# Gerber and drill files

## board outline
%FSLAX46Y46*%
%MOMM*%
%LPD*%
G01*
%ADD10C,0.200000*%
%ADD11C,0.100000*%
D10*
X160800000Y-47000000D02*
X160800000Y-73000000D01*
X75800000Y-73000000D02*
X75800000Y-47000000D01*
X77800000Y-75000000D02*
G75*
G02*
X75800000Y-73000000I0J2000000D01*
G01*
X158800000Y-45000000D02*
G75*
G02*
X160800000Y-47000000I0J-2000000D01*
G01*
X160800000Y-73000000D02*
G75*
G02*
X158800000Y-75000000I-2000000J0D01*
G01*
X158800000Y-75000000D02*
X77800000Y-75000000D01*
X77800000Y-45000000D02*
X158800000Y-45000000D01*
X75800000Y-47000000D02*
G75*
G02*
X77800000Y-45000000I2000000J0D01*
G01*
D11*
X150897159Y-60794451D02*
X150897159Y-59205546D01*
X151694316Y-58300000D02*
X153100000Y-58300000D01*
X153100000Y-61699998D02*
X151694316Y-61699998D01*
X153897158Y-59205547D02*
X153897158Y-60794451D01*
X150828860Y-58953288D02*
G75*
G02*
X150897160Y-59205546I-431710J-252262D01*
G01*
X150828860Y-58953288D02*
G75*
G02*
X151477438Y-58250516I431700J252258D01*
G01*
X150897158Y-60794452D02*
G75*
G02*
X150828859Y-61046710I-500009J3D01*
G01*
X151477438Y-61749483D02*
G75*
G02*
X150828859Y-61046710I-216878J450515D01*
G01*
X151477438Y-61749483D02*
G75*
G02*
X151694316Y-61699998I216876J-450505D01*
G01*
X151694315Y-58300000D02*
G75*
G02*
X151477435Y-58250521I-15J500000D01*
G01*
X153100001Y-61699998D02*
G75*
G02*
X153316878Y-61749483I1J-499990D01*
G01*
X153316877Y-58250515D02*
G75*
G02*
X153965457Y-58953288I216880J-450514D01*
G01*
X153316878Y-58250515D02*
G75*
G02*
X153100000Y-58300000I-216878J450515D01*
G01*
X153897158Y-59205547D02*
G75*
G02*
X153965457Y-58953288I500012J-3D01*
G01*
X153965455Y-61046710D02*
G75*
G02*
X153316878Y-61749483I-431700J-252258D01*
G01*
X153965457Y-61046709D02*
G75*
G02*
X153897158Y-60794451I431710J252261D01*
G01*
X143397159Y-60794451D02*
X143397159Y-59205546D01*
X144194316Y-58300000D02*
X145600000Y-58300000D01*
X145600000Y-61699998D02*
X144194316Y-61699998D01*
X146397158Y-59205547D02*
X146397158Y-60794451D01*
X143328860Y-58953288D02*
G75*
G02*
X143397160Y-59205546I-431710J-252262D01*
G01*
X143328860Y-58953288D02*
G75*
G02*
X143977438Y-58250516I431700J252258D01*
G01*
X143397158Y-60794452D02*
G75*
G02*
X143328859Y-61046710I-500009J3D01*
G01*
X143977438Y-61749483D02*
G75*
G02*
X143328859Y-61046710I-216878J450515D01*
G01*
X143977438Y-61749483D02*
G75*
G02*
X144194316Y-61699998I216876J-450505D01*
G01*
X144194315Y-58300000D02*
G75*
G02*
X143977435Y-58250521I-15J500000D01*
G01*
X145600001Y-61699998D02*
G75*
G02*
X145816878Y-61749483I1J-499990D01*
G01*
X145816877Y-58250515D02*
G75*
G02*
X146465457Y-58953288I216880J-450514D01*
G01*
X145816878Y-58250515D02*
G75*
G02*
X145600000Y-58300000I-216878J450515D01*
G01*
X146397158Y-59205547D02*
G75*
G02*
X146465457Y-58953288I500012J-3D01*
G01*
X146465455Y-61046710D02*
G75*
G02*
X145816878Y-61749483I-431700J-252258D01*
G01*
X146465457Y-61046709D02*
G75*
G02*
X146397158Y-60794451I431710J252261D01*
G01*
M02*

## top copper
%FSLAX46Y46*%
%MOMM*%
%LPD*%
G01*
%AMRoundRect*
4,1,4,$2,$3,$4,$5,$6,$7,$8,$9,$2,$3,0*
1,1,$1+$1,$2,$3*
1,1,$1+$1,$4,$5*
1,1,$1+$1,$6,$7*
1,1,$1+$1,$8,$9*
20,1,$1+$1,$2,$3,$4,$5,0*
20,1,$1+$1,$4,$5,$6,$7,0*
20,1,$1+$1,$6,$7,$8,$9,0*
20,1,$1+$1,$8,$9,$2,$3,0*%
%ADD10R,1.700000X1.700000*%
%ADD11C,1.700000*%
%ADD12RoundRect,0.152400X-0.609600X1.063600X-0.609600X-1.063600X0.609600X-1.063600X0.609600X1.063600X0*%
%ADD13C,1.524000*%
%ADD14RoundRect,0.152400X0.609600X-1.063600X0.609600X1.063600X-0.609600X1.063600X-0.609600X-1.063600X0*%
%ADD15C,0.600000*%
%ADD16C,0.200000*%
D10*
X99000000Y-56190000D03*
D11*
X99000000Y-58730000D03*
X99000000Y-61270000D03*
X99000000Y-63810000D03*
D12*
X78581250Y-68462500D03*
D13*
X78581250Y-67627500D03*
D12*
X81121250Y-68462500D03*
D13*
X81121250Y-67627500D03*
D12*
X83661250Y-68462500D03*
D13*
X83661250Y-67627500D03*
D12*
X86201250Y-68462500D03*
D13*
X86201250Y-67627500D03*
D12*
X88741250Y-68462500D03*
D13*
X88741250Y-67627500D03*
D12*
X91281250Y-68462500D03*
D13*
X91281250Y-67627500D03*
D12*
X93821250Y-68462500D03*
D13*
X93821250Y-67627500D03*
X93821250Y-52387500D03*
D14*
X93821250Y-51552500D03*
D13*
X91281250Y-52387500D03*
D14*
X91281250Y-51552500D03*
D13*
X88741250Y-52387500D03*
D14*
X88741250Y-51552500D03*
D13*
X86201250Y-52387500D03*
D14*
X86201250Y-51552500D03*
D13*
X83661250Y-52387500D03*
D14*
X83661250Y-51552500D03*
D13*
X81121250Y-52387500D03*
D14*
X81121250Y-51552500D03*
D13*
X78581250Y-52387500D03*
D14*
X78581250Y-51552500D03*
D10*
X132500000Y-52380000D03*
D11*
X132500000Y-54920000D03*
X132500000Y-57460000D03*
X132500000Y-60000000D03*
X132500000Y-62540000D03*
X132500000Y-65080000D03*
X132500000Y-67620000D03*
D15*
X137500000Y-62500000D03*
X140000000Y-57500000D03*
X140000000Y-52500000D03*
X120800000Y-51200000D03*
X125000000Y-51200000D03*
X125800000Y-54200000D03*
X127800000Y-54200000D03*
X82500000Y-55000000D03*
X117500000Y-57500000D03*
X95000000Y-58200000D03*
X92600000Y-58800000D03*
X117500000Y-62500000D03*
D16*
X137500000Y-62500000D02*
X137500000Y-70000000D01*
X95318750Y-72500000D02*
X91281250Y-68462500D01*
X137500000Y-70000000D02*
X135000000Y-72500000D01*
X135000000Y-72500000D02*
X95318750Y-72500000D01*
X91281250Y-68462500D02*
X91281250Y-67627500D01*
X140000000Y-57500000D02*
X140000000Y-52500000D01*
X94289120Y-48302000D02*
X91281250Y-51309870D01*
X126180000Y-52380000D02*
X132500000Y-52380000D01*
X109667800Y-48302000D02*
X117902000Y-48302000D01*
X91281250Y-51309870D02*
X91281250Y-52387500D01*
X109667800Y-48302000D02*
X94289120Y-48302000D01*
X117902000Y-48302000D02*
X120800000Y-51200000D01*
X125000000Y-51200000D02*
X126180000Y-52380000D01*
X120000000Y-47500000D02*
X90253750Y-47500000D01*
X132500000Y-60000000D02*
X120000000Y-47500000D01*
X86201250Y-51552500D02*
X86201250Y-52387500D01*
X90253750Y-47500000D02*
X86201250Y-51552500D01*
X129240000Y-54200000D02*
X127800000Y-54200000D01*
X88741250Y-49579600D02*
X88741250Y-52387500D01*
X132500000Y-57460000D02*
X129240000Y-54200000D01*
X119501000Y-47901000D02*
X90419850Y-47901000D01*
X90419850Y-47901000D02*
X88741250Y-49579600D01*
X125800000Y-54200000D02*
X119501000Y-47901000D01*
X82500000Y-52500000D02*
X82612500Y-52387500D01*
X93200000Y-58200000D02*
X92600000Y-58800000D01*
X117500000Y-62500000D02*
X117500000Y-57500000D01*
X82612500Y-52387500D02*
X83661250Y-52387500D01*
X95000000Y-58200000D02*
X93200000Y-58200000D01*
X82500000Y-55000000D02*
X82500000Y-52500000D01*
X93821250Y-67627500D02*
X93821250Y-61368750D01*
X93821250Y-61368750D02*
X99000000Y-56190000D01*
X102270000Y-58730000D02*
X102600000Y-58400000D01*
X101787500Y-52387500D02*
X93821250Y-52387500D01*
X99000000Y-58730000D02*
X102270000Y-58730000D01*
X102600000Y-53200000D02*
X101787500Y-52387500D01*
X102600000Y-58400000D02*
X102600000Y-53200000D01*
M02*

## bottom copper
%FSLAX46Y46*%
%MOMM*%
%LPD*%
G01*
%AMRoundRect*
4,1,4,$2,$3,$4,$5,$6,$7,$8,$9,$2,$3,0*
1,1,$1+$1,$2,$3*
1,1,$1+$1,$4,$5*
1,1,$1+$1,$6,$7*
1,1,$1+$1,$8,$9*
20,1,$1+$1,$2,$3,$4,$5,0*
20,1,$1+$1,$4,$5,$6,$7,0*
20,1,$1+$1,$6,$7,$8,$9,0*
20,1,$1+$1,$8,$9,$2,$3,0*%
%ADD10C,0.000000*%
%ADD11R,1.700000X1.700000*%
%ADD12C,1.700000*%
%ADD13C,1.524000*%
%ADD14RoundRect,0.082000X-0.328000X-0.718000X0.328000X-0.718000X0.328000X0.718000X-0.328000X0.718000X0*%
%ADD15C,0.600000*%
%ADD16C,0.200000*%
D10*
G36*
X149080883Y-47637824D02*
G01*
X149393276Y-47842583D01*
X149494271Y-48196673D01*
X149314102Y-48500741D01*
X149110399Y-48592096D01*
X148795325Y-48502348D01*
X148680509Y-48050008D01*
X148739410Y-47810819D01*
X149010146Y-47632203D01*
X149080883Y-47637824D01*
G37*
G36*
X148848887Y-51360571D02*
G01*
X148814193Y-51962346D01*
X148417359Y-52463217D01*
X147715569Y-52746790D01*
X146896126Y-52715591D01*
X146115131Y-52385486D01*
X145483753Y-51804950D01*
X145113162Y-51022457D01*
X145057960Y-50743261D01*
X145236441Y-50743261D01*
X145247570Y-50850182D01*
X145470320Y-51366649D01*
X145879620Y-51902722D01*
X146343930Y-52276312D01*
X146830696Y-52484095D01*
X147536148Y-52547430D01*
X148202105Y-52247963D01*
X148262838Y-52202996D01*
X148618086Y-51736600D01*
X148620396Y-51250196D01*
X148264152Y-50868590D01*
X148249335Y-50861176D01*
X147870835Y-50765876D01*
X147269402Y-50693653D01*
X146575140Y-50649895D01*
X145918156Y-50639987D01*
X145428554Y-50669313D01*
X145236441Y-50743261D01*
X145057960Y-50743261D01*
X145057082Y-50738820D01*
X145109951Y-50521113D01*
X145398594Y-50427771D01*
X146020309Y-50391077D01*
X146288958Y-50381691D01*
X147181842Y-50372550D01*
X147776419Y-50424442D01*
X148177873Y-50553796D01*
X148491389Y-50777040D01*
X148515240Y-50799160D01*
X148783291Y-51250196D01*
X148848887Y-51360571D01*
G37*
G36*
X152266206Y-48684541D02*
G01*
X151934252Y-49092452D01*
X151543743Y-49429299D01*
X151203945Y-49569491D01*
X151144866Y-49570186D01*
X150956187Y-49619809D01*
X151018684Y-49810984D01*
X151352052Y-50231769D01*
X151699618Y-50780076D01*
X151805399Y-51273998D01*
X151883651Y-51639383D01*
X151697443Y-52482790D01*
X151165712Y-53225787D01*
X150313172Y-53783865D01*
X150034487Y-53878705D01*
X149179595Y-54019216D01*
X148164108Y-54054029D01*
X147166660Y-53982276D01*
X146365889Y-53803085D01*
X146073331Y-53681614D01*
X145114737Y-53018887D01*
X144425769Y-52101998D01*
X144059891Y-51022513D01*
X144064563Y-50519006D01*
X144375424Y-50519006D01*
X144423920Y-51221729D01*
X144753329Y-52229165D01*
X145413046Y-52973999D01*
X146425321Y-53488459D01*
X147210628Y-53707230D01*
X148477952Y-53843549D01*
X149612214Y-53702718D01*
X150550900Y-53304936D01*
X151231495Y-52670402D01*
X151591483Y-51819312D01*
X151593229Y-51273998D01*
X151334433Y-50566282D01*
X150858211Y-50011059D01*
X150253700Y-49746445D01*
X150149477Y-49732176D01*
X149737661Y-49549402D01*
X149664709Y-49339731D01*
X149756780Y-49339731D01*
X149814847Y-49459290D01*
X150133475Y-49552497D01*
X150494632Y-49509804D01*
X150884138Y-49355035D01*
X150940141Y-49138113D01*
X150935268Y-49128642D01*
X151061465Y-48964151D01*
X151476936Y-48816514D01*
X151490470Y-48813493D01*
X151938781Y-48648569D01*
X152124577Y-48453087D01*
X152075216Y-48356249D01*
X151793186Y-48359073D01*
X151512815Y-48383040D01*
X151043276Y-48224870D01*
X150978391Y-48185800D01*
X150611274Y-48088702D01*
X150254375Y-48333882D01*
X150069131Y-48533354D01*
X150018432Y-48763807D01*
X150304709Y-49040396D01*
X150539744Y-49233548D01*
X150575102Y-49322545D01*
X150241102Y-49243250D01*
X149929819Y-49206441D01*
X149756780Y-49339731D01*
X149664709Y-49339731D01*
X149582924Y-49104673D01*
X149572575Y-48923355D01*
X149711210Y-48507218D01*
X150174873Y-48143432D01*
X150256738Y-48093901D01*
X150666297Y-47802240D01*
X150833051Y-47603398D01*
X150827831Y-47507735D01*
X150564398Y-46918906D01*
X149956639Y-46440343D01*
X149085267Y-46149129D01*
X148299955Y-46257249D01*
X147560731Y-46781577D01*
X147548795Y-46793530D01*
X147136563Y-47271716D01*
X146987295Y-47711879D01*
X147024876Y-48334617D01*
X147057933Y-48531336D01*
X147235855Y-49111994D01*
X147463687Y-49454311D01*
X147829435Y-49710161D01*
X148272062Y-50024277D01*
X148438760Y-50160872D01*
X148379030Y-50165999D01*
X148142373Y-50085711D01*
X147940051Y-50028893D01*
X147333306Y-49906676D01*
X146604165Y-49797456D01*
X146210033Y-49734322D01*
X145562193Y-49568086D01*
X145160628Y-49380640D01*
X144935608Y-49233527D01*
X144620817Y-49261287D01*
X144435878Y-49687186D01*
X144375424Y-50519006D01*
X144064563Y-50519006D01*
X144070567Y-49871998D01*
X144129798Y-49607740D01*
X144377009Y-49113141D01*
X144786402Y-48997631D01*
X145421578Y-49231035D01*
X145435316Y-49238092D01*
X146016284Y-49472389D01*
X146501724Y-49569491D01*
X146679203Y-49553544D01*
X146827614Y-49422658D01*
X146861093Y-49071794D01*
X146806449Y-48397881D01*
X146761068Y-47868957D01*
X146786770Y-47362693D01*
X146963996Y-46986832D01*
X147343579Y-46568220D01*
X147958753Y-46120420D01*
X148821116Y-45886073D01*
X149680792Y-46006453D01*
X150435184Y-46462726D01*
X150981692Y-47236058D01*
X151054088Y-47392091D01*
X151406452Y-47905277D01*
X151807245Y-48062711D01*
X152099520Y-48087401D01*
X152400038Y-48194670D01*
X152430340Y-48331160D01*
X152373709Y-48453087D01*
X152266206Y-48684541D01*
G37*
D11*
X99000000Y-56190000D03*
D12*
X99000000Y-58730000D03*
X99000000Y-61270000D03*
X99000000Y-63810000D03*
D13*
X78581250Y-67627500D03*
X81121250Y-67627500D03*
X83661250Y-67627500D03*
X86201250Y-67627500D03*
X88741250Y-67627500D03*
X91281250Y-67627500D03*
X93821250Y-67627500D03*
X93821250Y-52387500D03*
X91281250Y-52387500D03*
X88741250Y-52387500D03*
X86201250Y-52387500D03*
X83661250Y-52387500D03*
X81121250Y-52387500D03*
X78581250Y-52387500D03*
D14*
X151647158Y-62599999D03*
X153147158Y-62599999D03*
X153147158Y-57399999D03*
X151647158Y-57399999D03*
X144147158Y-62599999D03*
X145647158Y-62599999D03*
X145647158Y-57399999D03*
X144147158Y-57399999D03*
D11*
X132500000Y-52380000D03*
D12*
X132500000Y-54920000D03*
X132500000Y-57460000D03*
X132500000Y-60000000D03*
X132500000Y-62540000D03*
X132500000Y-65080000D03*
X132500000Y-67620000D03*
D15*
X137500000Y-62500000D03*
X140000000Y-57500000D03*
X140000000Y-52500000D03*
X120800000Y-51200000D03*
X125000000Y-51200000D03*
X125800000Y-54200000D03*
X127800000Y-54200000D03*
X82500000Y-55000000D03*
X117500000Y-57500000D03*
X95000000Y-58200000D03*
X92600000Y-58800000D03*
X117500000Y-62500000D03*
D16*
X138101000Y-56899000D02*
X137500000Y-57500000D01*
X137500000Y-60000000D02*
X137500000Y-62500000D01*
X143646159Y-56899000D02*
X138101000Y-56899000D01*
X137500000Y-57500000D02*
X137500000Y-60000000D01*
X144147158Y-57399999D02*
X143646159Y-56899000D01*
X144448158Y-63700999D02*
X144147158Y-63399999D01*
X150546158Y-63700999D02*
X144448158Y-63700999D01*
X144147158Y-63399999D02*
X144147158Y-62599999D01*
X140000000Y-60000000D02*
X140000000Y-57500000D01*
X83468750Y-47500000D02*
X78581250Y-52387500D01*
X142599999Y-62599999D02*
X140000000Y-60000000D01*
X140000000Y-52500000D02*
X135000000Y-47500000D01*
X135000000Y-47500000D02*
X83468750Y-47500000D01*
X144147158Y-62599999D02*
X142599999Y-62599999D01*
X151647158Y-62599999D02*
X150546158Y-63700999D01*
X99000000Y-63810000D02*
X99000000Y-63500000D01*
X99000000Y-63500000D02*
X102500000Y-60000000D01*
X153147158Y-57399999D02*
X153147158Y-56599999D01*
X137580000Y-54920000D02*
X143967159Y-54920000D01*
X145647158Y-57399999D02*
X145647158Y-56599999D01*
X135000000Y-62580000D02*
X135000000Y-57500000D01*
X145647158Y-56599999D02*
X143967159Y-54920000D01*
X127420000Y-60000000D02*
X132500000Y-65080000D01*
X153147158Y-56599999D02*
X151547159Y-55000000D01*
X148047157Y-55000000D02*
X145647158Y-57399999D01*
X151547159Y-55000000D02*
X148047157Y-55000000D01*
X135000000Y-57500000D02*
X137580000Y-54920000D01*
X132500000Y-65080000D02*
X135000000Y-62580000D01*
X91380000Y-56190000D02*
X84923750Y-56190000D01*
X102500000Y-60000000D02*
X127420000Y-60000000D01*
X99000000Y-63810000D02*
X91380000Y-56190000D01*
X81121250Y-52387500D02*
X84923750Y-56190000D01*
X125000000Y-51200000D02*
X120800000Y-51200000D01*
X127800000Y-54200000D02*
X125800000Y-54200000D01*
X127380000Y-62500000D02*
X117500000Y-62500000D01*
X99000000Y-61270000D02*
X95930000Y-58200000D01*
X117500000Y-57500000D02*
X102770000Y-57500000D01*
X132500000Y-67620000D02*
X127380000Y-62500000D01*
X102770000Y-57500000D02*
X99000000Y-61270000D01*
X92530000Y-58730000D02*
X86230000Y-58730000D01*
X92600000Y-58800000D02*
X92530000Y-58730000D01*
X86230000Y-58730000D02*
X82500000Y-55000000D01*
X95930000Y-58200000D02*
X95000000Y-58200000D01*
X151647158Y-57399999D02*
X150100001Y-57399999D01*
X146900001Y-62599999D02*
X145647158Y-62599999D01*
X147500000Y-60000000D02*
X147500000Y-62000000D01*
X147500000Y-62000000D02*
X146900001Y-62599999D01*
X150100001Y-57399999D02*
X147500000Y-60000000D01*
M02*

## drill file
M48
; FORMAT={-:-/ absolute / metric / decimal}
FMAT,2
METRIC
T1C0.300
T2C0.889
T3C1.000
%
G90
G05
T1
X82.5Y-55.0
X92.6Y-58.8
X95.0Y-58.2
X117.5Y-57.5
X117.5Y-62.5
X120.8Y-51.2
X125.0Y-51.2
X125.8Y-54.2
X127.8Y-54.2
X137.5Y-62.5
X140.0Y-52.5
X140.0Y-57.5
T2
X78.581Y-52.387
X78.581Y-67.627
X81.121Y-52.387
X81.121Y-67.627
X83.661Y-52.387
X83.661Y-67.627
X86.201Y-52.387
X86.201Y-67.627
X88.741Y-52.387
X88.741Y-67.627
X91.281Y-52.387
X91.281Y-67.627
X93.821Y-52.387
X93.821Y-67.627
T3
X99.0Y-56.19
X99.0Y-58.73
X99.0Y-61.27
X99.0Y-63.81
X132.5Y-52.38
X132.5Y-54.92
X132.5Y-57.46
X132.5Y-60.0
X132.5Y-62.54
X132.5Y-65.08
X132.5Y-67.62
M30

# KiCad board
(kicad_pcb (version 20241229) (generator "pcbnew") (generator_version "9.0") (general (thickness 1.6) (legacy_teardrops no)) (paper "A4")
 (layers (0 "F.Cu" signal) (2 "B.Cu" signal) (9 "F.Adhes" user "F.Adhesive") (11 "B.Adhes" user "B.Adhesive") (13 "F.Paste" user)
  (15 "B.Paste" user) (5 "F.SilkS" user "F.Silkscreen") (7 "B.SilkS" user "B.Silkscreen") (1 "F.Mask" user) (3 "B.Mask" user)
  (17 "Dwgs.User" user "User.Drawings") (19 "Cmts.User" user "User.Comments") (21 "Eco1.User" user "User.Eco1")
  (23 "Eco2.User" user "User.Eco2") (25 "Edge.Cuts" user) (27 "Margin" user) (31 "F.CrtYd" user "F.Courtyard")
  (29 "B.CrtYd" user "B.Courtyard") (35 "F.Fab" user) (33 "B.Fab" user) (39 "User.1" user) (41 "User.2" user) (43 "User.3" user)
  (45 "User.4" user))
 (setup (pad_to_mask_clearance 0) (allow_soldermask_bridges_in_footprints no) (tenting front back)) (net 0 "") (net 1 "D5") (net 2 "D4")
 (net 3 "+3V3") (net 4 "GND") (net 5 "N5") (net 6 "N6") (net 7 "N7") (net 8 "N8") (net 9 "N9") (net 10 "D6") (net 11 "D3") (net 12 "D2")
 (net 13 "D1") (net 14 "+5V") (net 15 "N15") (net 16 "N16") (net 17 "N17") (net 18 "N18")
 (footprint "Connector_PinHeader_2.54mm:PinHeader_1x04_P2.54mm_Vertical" (layer "F.Cu") (at 99 56.19)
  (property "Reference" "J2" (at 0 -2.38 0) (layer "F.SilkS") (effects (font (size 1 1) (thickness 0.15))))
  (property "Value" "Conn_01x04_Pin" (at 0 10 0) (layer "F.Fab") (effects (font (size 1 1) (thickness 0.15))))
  (pad "1" thru_hole rect (at 0 0) (size 1.7 1.7) (drill 1) (layers "*.Cu" "*.Mask") (remove_unused_layers no) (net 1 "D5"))
  (pad "2" thru_hole circle (at 0 2.54) (size 1.7 1.7) (drill 1) (layers "*.Cu" "*.Mask") (remove_unused_layers no) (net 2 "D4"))
  (pad "3" thru_hole circle (at 0 5.08) (size 1.7 1.7) (drill 1) (layers "*.Cu" "*.Mask") (remove_unused_layers no) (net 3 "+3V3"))
  (pad "4" thru_hole circle (at 0 7.62) (size 1.7 1.7) (drill 1) (layers "*.Cu" "*.Mask") (remove_unused_layers no) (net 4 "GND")))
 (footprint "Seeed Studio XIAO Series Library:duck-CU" (layer "F.Cu") (at 148.25 50)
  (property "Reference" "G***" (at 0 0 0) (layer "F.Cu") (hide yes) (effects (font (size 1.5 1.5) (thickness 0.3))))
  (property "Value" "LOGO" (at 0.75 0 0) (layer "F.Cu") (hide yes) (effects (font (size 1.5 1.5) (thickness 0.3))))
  (fp_poly
   (pts (xy 0.48941 -2.189181) (xy 0.430509 -1.949992) (xy 0.545325 -1.497652) (xy 0.860399 -1.407904) (xy 1.064102 -1.499259)
    (xy 1.244271 -1.803327) (xy 1.143276 -2.157417) (xy 0.830883 -2.362176) (xy 0.760146 -2.367797))
   (stroke (width 0) (type solid)) (fill yes) (layer "B.Cu"))
  (fp_poly
   (pts (xy -1.961042 0.381691) (xy -2.229691 0.391077) (xy -2.851406 0.427771) (xy -3.140049 0.521113) (xy -3.192918 0.73882)
    (xy -3.136838 1.022457) (xy -2.766247 1.80495) (xy -2.134869 2.385486) (xy -1.353874 2.715591) (xy -0.534431 2.74679)
    (xy 0.167359 2.463217) (xy 0.564193 1.962346) (xy 0.598887 1.360571) (xy 0.533291 1.250196) (xy 0.370396 1.250196) (xy 0.368086 1.7366)
    (xy 0.012838 2.202996) (xy -0.047895 2.247963) (xy -0.713852 2.54743) (xy -1.419304 2.484095) (xy -1.90607 2.276312)
    (xy -2.37038 1.902722) (xy -2.77968 1.366649) (xy -3.00243 0.850182) (xy -3.013559 0.743261) (xy -2.821446 0.669313)
    (xy -2.331844 0.639987) (xy -1.67486 0.649895) (xy -0.980598 0.693653) (xy -0.379165 0.765876) (xy -0.000665 0.861176)
    (xy 0.014152 0.86859) (xy 0.370396 1.250196) (xy 0.533291 1.250196) (xy 0.26524 0.79916) (xy 0.241389 0.77704) (xy -0.072127 0.553796)
    (xy -0.473581 0.424442) (xy -1.068158 0.37255))
   (stroke (width 0) (type solid)) (fill yes) (layer "B.Cu"))
  (fp_poly
   (pts (xy -0.291247 -3.87958) (xy -0.906421 -3.43178) (xy -1.286004 -3.013168) (xy -1.46323 -2.637307) (xy -1.488932 -2.131043)
    (xy -1.443551 -1.602119) (xy -1.388907 -0.928206) (xy -1.422386 -0.577342) (xy -1.570797 -0.446456) (xy -1.748276 -0.430509)
    (xy -2.233716 -0.527611) (xy -2.814684 -0.761908) (xy -2.828422 -0.768965) (xy -3.463598 -1.002369) (xy -3.872991 -0.886859)
    (xy -4.120202 -0.39226) (xy -4.179433 -0.128002) (xy -4.190109 1.022513) (xy -3.824231 2.101998) (xy -3.135263 3.018887)
    (xy -2.176669 3.681614) (xy -1.884111 3.803085) (xy -1.08334 3.982276) (xy -0.085892 4.054029) (xy 0.929595 4.019216)
    (xy 1.784487 3.878705) (xy 2.063172 3.783865) (xy 2.915712 3.225787) (xy 3.447443 2.48279) (xy 3.633651 1.639383) (xy 3.555399 1.273998)
    (xy 3.343229 1.273998) (xy 3.341483 1.819312) (xy 2.981495 2.670402) (xy 2.3009 3.304936) (xy 1.362214 3.702718) (xy 0.227952 3.843549)
    (xy -1.039372 3.70723) (xy -1.824679 3.488459) (xy -2.836954 2.973999) (xy -3.496671 2.229165) (xy -3.82608 1.221729)
    (xy -3.874576 0.519006) (xy -3.814122 -0.312814) (xy -3.629183 -0.738713) (xy -3.314392 -0.766473) (xy -3.089372 -0.61936)
    (xy -2.687807 -0.431914) (xy -2.039967 -0.265678) (xy -1.645835 -0.202544) (xy -0.916694 -0.093324) (xy -0.309949 0.028893)
    (xy -0.107627 0.085711) (xy 0.12903 0.165999) (xy 0.18876 0.160872) (xy 0.022062 0.024277) (xy -0.420565 -0.289839)
    (xy -0.786313 -0.545689) (xy -1.014145 -0.888006) (xy -1.192067 -1.468664) (xy -1.225124 -1.665383) (xy -1.262705 -2.288121)
    (xy -1.113437 -2.728284) (xy -0.701205 -3.20647) (xy -0.689269 -3.218423) (xy 0.049955 -3.742751) (xy 0.835267 -3.850871)
    (xy 1.706639 -3.559657) (xy 2.314398 -3.081094) (xy 2.577831 -2.492265) (xy 2.583051 -2.396602) (xy 2.416297 -2.19776)
    (xy 2.006738 -1.906099) (xy 1.924873 -1.856568) (xy 1.46121 -1.492782) (xy 1.322575 -1.076645) (xy 1.332924 -0.895327)
    (xy 1.487661 -0.450598) (xy 1.899477 -0.267824) (xy 2.0037 -0.253555) (xy 2.608211 0.011059) (xy 3.084433 0.566282)
    (xy 3.343229 1.273998) (xy 3.555399 1.273998) (xy 3.449618 0.780076) (xy 3.102052 0.231769) (xy 2.768684 -0.189016)
    (xy 2.706187 -0.380191) (xy 2.894866 -0.429814) (xy 2.953945 -0.430509) (xy 3.293743 -0.570701) (xy 3.684252 -0.907548)
    (xy 4.016206 -1.315459) (xy 4.123709 -1.546913) (xy 3.874577 -1.546913) (xy 3.688781 -1.351431) (xy 3.24047 -1.186507)
    (xy 3.226936 -1.183486) (xy 2.811465 -1.035849) (xy 2.685268 -0.871358) (xy 2.690141 -0.861887) (xy 2.634138 -0.644965)
    (xy 2.244632 -0.490196) (xy 1.883475 -0.447503) (xy 1.564847 -0.54071) (xy 1.50678 -0.660269) (xy 1.679819 -0.793559)
    (xy 1.991102 -0.75675) (xy 2.325102 -0.677455) (xy 2.289744 -0.766452) (xy 2.054709 -0.959604) (xy 1.768432 -1.236193)
    (xy 1.819131 -1.466646) (xy 2.004375 -1.666118) (xy 2.361274 -1.911298) (xy 2.728391 -1.8142) (xy 2.793276 -1.77513)
    (xy 3.262815 -1.61696) (xy 3.543186 -1.640927) (xy 3.825216 -1.643751) (xy 3.874577 -1.546913) (xy 4.123709 -1.546913)
    (xy 4.18034 -1.66884) (xy 4.150038 -1.80533) (xy 3.84952 -1.912599) (xy 3.557245 -1.937289) (xy 3.156452 -2.094723)
    (xy 2.804088 -2.607909) (xy 2.731692 -2.763942) (xy 2.185184 -3.537274) (xy 1.430792 -3.993547) (xy 0.571116 -4.113927))
   (stroke (width 0) (type solid)) (fill yes) (layer "B.Cu")))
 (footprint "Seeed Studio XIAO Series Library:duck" (layer "F.Cu") (at 148 50)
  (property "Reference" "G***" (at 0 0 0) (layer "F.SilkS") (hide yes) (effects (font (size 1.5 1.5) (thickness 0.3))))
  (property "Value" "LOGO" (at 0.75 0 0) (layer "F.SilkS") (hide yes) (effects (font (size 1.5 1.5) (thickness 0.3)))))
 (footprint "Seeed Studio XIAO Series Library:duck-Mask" (layer "F.Cu") (at 148.25 50)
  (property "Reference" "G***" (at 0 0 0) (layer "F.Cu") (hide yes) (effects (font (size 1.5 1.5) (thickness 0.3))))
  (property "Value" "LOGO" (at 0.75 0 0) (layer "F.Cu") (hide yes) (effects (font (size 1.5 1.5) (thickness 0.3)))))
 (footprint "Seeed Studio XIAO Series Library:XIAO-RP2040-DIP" (layer "F.Cu") (at 86.20125 60.0075 90)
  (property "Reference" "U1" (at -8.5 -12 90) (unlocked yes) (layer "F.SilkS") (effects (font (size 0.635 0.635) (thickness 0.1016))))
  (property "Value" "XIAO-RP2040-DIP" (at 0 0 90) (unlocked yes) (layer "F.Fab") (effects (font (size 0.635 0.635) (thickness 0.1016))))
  (pad "1" smd roundrect (at -8.455 -7.62 270) (size 2.432 1.524) (layers "F.Cu" "F.Mask") (roundrect_rratio 0.1) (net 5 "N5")
   (thermal_bridge_angle 45))
  (pad "1" thru_hole circle (at -7.62 -7.62 270) (size 1.524 1.524) (drill 0.889) (layers "*.Cu" "*.Mask") (remove_unused_layers no)
   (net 5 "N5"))
  (pad "2" smd roundrect (at -8.455 -5.08 270) (size 2.432 1.524) (layers "F.Cu" "F.Mask") (roundrect_rratio 0.1) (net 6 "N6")
   (thermal_bridge_angle 45))
  (pad "2" thru_hole circle (at -7.62 -5.08 270) (size 1.524 1.524) (drill 0.889) (layers "*.Cu" "*.Mask") (remove_unused_layers no)
   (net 6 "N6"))
  (pad "3" smd roundrect (at -8.455 -2.54 270) (size 2.432 1.524) (layers "F.Cu" "F.Mask") (roundrect_rratio 0.1) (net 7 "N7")
   (thermal_bridge_angle 45))
  (pad "3" thru_hole circle (at -7.62 -2.54 270) (size 1.524 1.524) (drill 0.889) (layers "*.Cu" "*.Mask") (remove_unused_layers no)
   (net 7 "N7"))
  (pad "4" smd roundrect (at -8.455 0 270) (size 2.432 1.524) (layers "F.Cu" "F.Mask") (roundrect_rratio 0.1) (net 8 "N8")
   (thermal_bridge_angle 45))
  (pad "4" thru_hole circle (at -7.62 0 270) (size 1.524 1.524) (drill 0.889) (layers "*.Cu" "*.Mask") (remove_unused_layers no)
   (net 8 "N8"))
  (pad "5" smd roundrect (at -8.455 2.54 270) (size 2.432 1.524) (layers "F.Cu" "F.Mask") (roundrect_rratio 0.1) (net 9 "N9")
   (thermal_bridge_angle 45))
  (pad "5" thru_hole circle (at -7.62 2.54 270) (size 1.524 1.524) (drill 0.889) (layers "*.Cu" "*.Mask") (remove_unused_layers no)
   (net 9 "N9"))
  (pad "6" smd roundrect (at -8.455 5.08 270) (size 2.432 1.524) (layers "F.Cu" "F.Mask") (roundrect_rratio 0.1) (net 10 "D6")
   (thermal_bridge_angle 45))
  (pad "6" thru_hole circle (at -7.62 5.08 270) (size 1.524 1.524) (drill 0.889) (layers "*.Cu" "*.Mask") (remove_unused_layers no)
   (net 10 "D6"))
  (pad "7" smd roundrect (at -8.455 7.62 270) (size 2.432 1.524) (layers "F.Cu" "F.Mask") (roundrect_rratio 0.1) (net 1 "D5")
   (thermal_bridge_angle 45))
  (pad "7" thru_hole circle (at -7.62 7.62 270) (size 1.524 1.524) (drill 0.889) (layers "*.Cu" "*.Mask") (remove_unused_layers no)
   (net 1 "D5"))
  (pad "8" thru_hole circle (at 7.62 7.62 90) (size 1.524 1.524) (drill 0.889) (layers "*.Cu" "*.Mask") (remove_unused_layers no)
   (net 2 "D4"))
  (pad "8" smd roundrect (at 8.455 7.62 90) (size 2.432 1.524) (layers "F.Cu" "F.Mask") (roundrect_rratio 0.1) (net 2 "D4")
   (thermal_bridge_angle 45))
  (pad "9" thru_hole circle (at 7.62 5.08 90) (size 1.524 1.524) (drill 0.889) (layers "*.Cu" "*.Mask") (remove_unused_layers no)
   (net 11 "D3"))
  (pad "9" smd roundrect (at 8.455 5.08 90) (size 2.432 1.524) (layers "F.Cu" "F.Mask") (roundrect_rratio 0.1) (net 11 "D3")
   (thermal_bridge_angle 45))
  (pad "10" thru_hole circle (at 7.62 2.54 90) (size 1.524 1.524) (drill 0.889) (layers "*.Cu" "*.Mask") (remove_unused_layers no)
   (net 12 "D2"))
  (pad "10" smd roundrect (at 8.455 2.54 90) (size 2.432 1.524) (layers "F.Cu" "F.Mask") (roundrect_rratio 0.1) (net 12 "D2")
   (thermal_bridge_angle 45))
  (pad "11" thru_hole circle (at 7.62 0 90) (size 1.524 1.524) (drill 0.889) (layers "*.Cu" "*.Mask") (remove_unused_layers no)
   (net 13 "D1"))
  (pad "11" smd roundrect (at 8.455 0 90) (size 2.432 1.524) (layers "F.Cu" "F.Mask") (roundrect_rratio 0.1) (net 13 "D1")
   (thermal_bridge_angle 45))
  (pad "12" thru_hole circle (at 7.62 -2.54 90) (size 1.524 1.524) (drill 0.889) (layers "*.Cu" "*.Mask") (remove_unused_layers no)
   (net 3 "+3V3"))
  (pad "12" smd roundrect (at 8.455 -2.54 90) (size 2.432 1.524) (layers "F.Cu" "F.Mask") (roundrect_rratio 0.1) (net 3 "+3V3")
   (thermal_bridge_angle 45))
  (pad "13" thru_hole circle (at 7.62 -5.08 90) (size 1.524 1.524) (drill 0.889) (layers "*.Cu" "*.Mask") (remove_unused_layers no)
   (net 4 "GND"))
  (pad "13" smd roundrect (at 8.455 -5.08 90) (size 2.432 1.524) (layers "F.Cu" "F.Mask") (roundrect_rratio 0.1) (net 4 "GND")
   (thermal_bridge_angle 45))
  (pad "14" thru_hole circle (at 7.62 -7.62 90) (size 1.524 1.524) (drill 0.889) (layers "*.Cu" "*.Mask") (remove_unused_layers no)
   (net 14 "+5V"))
  (pad "14" smd roundrect (at 8.455 -7.62 90) (size 2.432 1.524) (layers "F.Cu" "F.Mask") (roundrect_rratio 0.1) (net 14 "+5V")
   (thermal_bridge_angle 45)))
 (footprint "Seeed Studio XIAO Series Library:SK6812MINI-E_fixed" (layer "F.Cu") (at 152.5 60 90)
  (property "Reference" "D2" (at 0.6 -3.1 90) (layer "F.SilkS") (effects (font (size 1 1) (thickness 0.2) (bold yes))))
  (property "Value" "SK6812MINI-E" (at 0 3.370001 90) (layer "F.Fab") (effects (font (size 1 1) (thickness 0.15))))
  (fp_line (start -0.794451 -1.602841) (end 0.794454 -1.602841) (stroke (width 0.1) (type solid)) (layer "Edge.Cuts"))
  (fp_line (start 1.7 -0.805684) (end 1.7 0.6) (stroke (width 0.1) (type solid)) (layer "Edge.Cuts"))
  (fp_line (start -1.699998 0.6) (end -1.699998 -0.805684) (stroke (width 0.1) (type solid)) (layer "Edge.Cuts"))
  (fp_line (start 0.794453 1.397158) (end -0.794451 1.397158) (stroke (width 0.1) (type solid)) (layer "Edge.Cuts"))
  (fp_arc (start 1.046712 -1.67114) (mid 0.925124 -1.620218) (end 0.794454 -1.602841) (stroke (width 0.1) (type solid)) (layer "Edge.Cuts"))
  (fp_arc (start 1.046712 -1.67114) (mid 1.638072 -1.606876) (end 1.749485 -1.022562) (stroke (width 0.1) (type solid)) (layer "Edge.Cuts"))
  (fp_arc (start -0.794452 -1.602842) (mid -0.925122 -1.620219) (end -1.04671 -1.671141) (stroke (width 0.1) (type solid))
   (layer "Edge.Cuts"))
  (fp_arc (start -1.749483 -1.022562) (mid -1.63807 -1.606877) (end -1.04671 -1.671141) (stroke (width 0.1) (type solid))
   (layer "Edge.Cuts"))
  (fp_arc (start -1.749483 -1.022562) (mid -1.712526 -0.91691) (end -1.699998 -0.805684) (stroke (width 0.1) (type solid))
   (layer "Edge.Cuts"))
  (fp_arc (start 1.7 -0.805685) (mid 1.712528 -0.91691) (end 1.749485 -1.022562) (stroke (width 0.1) (type solid)) (layer "Edge.Cuts"))
  (fp_arc (start -1.699998 0.600001) (mid -1.712526 0.711226) (end -1.749483 0.816878) (stroke (width 0.1) (type solid)) (layer "Edge.Cuts"))
  (fp_arc (start 1.749485 0.816877) (mid 1.638073 1.401193) (end 1.046712 1.465457) (stroke (width 0.1) (type solid)) (layer "Edge.Cuts"))
  (fp_arc (start 1.749485 0.816878) (mid 1.712528 0.711226) (end 1.7 0.6) (stroke (width 0.1) (type solid)) (layer "Edge.Cuts"))
  (fp_arc (start 0.794453 1.397158) (mid 0.925124 1.414535) (end 1.046712 1.465457) (stroke (width 0.1) (type solid)) (layer "Edge.Cuts"))
  (fp_arc (start -1.04671 1.465455) (mid -1.638069 1.401192) (end -1.749483 0.816878) (stroke (width 0.1) (type solid)) (layer "Edge.Cuts"))
  (fp_arc (start -1.046709 1.465457) (mid -0.925121 1.414535) (end -0.794451 1.397158) (stroke (width 0.1) (type solid)) (layer "Edge.Cuts"))
  (pad "1" smd roundrect (at -2.599999 -0.852842) (size 0.82 1.6) (layers "B.Cu" "B.Mask" "B.Paste") (roundrect_rratio 0.1) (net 14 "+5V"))
  (pad "2" smd roundrect (at -2.599999 0.647158) (size 0.82 1.6) (layers "B.Cu" "B.Mask" "B.Paste") (roundrect_rratio 0.1) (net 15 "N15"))
  (pad "3" smd roundrect (at 2.600001 0.647158) (size 0.82 1.6) (layers "B.Cu" "B.Mask" "B.Paste") (roundrect_rratio 0.1) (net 4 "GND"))
  (pad "4" smd roundrect (at 2.600001 -0.852842) (size 0.82 1.6) (layers "B.Cu" "B.Mask" "B.Paste") (roundrect_rratio 0.1) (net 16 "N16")))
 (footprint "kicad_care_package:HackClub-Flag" (layer "F.Cu") (at 148 69)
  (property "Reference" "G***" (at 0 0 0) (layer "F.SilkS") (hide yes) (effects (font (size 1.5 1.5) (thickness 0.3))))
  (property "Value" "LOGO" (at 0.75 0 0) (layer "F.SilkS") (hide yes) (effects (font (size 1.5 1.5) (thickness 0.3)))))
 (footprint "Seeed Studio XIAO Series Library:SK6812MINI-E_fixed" (layer "F.Cu") (at 145 60 90)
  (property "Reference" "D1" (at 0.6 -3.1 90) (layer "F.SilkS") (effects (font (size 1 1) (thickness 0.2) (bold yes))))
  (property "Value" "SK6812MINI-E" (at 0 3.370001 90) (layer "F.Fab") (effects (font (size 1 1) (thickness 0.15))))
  (fp_line (start -0.794451 -1.602841) (end 0.794454 -1.602841) (stroke (width 0.1) (type solid)) (layer "Edge.Cuts"))
  (fp_line (start 1.7 -0.805684) (end 1.7 0.6) (stroke (width 0.1) (type solid)) (layer "Edge.Cuts"))
  (fp_line (start -1.699998 0.6) (end -1.699998 -0.805684) (stroke (width 0.1) (type solid)) (layer "Edge.Cuts"))
  (fp_line (start 0.794453 1.397158) (end -0.794451 1.397158) (stroke (width 0.1) (type solid)) (layer "Edge.Cuts"))
  (fp_arc (start 1.046712 -1.67114) (mid 0.925124 -1.620218) (end 0.794454 -1.602841) (stroke (width 0.1) (type solid)) (layer "Edge.Cuts"))
  (fp_arc (start 1.046712 -1.67114) (mid 1.638072 -1.606876) (end 1.749485 -1.022562) (stroke (width 0.1) (type solid)) (layer "Edge.Cuts"))
  (fp_arc (start -0.794452 -1.602842) (mid -0.925122 -1.620219) (end -1.04671 -1.671141) (stroke (width 0.1) (type solid))
   (layer "Edge.Cuts"))
  (fp_arc (start -1.749483 -1.022562) (mid -1.63807 -1.606877) (end -1.04671 -1.671141) (stroke (width 0.1) (type solid))
   (layer "Edge.Cuts"))
  (fp_arc (start -1.749483 -1.022562) (mid -1.712526 -0.91691) (end -1.699998 -0.805684) (stroke (width 0.1) (type solid))
   (layer "Edge.Cuts"))
  (fp_arc (start 1.7 -0.805685) (mid 1.712528 -0.91691) (end 1.749485 -1.022562) (stroke (width 0.1) (type solid)) (layer "Edge.Cuts"))
  (fp_arc (start -1.699998 0.600001) (mid -1.712526 0.711226) (end -1.749483 0.816878) (stroke (width 0.1) (type solid)) (layer "Edge.Cuts"))
  (fp_arc (start 1.749485 0.816877) (mid 1.638073 1.401193) (end 1.046712 1.465457) (stroke (width 0.1) (type solid)) (layer "Edge.Cuts"))
  (fp_arc (start 1.749485 0.816878) (mid 1.712528 0.711226) (end 1.7 0.6) (stroke (width 0.1) (type solid)) (layer "Edge.Cuts"))
  (fp_arc (start 0.794453 1.397158) (mid 0.925124 1.414535) (end 1.046712 1.465457) (stroke (width 0.1) (type solid)) (layer "Edge.Cuts"))
  (fp_arc (start -1.04671 1.465455) (mid -1.638069 1.401192) (end -1.749483 0.816878) (stroke (width 0.1) (type solid)) (layer "Edge.Cuts"))
  (fp_arc (start -1.046709 1.465457) (mid -0.925121 1.414535) (end -0.794451 1.397158) (stroke (width 0.1) (type solid)) (layer "Edge.Cuts"))
  (pad "1" smd roundrect (at -2.599999 -0.852842) (size 0.82 1.6) (layers "B.Cu" "B.Mask" "B.Paste") (roundrect_rratio 0.1) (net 14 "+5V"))
  (pad "2" smd roundrect (at -2.599999 0.647158) (size 0.82 1.6) (layers "B.Cu" "B.Mask" "B.Paste") (roundrect_rratio 0.1) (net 16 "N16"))
  (pad "3" smd roundrect (at 2.600001 0.647158) (size 0.82 1.6) (layers "B.Cu" "B.Mask" "B.Paste") (roundrect_rratio 0.1) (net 4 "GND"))
  (pad "4" smd roundrect (at 2.600001 -0.852842) (size 0.82 1.6) (layers "B.Cu" "B.Mask" "B.Paste") (roundrect_rratio 0.1) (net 10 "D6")))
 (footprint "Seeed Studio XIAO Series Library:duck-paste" (layer "F.Cu") (at 148.25 50)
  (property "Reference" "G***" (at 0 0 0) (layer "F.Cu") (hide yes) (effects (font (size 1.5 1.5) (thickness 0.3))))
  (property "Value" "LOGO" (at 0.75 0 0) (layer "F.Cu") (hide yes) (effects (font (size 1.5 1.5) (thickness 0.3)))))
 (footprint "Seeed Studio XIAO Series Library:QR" (layer "B.Cu") (at 106 66 180)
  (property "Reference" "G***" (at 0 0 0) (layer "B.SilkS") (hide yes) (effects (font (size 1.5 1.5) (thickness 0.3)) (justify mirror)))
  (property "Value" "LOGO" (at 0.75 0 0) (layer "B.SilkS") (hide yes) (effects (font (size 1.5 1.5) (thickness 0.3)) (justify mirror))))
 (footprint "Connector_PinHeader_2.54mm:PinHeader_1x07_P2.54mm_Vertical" (layer "B.Cu") (at 132.5 52.38 180)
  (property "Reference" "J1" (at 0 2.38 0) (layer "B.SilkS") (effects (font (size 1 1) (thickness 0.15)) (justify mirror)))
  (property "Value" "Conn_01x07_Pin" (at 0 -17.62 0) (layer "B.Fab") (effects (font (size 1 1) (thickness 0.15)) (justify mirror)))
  (pad "1" thru_hole rect (at 0 0 180) (size 1.7 1.7) (drill 1) (layers "*.Cu" "*.Mask") (remove_unused_layers no) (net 11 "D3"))
  (pad "2" thru_hole circle (at 0 -2.54 180) (size 1.7 1.7) (drill 1) (layers "*.Cu" "*.Mask") (remove_unused_layers no) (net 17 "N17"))
  (pad "3" thru_hole circle (at 0 -5.08 180) (size 1.7 1.7) (drill 1) (layers "*.Cu" "*.Mask") (remove_unused_layers no) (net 12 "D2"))
  (pad "4" thru_hole circle (at 0 -7.62 180) (size 1.7 1.7) (drill 1) (layers "*.Cu" "*.Mask") (remove_unused_layers no) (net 13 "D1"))
  (pad "5" thru_hole circle (at 0 -10.16 180) (size 1.7 1.7) (drill 1) (layers "*.Cu" "*.Mask") (remove_unused_layers no) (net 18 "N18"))
  (pad "6" thru_hole circle (at 0 -12.7 180) (size 1.7 1.7) (drill 1) (layers "*.Cu" "*.Mask") (remove_unused_layers no) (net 4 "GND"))
  (pad "7" thru_hole circle (at 0 -15.24 180) (size 1.7 1.7) (drill 1) (layers "*.Cu" "*.Mask") (remove_unused_layers no) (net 3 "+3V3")))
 (gr_line (start 160.8 47) (end 160.8 73) (stroke (width 0.2) (type default)) (layer "Edge.Cuts"))
 (gr_line (start 75.8 73) (end 75.8 47) (stroke (width 0.2) (type default)) (layer "Edge.Cuts"))
 (gr_arc (start 77.8 75) (mid 76.385786 74.414214) (end 75.8 73) (stroke (width 0.2) (type default)) (layer "Edge.Cuts"))
 (gr_arc (start 158.8 45) (mid 160.214214 45.585786) (end 160.8 47) (stroke (width 0.2) (type default)) (layer "Edge.Cuts"))
 (gr_arc (start 160.8 73) (mid 160.214214 74.414214) (end 158.8 75) (stroke (width 0.2) (type default)) (layer "Edge.Cuts"))
 (gr_line (start 158.8 75) (end 77.8 75) (stroke (width 0.2) (type default)) (layer "Edge.Cuts"))
 (gr_line (start 77.8 45) (end 158.8 45) (stroke (width 0.2) (type default)) (layer "Edge.Cuts"))
 (gr_arc (start 75.8 47) (mid 76.385786 45.585786) (end 77.8 45) (stroke (width 0.2) (type default)) (layer "Edge.Cuts"))
 (segment (start 137.5 62.5) (end 137.5 70) (width 0.2) (layer "F.Cu") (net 10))
 (segment (start 95.31875 72.5) (end 91.28125 68.4625) (width 0.2) (layer "F.Cu") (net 10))
 (segment (start 137.5 70) (end 135 72.5) (width 0.2) (layer "F.Cu") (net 10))
 (segment (start 135 72.5) (end 95.31875 72.5) (width 0.2) (layer "F.Cu") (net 10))
 (segment (start 91.28125 68.4625) (end 91.28125 67.6275) (width 0.2) (layer "F.Cu") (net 10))
 (via (at 137.5 62.5) (size 0.6) (drill 0.3) (layers "F.Cu" "B.Cu") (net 10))
 (segment (start 138.101 56.899) (end 137.5 57.5) (width 0.2) (layer "B.Cu") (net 10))
 (segment (start 137.5 60) (end 137.5 62.5) (width 0.2) (layer "B.Cu") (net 10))
 (segment (start 143.646159 56.899) (end 138.101 56.899) (width 0.2) (layer "B.Cu") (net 10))
 (segment (start 137.5 57.5) (end 137.5 60) (width 0.2) (layer "B.Cu") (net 10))
 (segment (start 144.147158 57.399999) (end 143.646159 56.899) (width 0.2) (layer "B.Cu") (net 10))
 (segment (start 140 57.5) (end 140 52.5) (width 0.2) (layer "F.Cu") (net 14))
 (via (at 140 57.5) (size 0.6) (drill 0.3) (layers "F.Cu" "B.Cu") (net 14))
 (via (at 140 52.5) (size 0.6) (drill 0.3) (layers "F.Cu" "B.Cu") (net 14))
 (segment (start 144.448158 63.700999) (end 144.147158 63.399999) (width 0.2) (layer "B.Cu") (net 14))
 (segment (start 150.546158 63.700999) (end 144.448158 63.700999) (width 0.2) (layer "B.Cu") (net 14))
 (segment (start 144.147158 63.399999) (end 144.147158 62.599999) (width 0.2) (layer "B.Cu") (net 14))
 (segment (start 140 60) (end 140 57.5) (width 0.2) (layer "B.Cu") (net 14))
 (segment (start 83.46875 47.5) (end 78.58125 52.3875) (width 0.2) (layer "B.Cu") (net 14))
 (segment (start 142.599999 62.599999) (end 140 60) (width 0.2) (layer "B.Cu") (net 14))
 (segment (start 140 52.5) (end 135 47.5) (width 0.2) (layer "B.Cu") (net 14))
 (segment (start 135 47.5) (end 83.46875 47.5) (width 0.2) (layer "B.Cu") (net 14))
 (segment (start 144.147158 62.599999) (end 142.599999 62.599999) (width 0.2) (layer "B.Cu") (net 14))
 (segment (start 151.647158 62.599999) (end 150.546158 63.700999) (width 0.2) (layer "B.Cu") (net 14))
 (segment (start 99 63.81) (end 99 63.5) (width 0.2) (layer "B.Cu") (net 4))
 (segment (start 99 63.5) (end 102.5 60) (width 0.2) (layer "B.Cu") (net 4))
 (segment (start 153.147158 57.399999) (end 153.147158 56.599999) (width 0.2) (layer "B.Cu") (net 4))
 (segment (start 137.58 54.92) (end 143.967159 54.92) (width 0.2) (layer "B.Cu") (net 4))
 (segment (start 145.647158 57.399999) (end 145.647158 56.599999) (width 0.2) (layer "B.Cu") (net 4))
 (segment (start 135 62.58) (end 135 57.5) (width 0.2) (layer "B.Cu") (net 4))
 (segment (start 145.647158 56.599999) (end 143.967159 54.92) (width 0.2) (layer "B.Cu") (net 4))
 (segment (start 127.42 60) (end 132.5 65.08) (width 0.2) (layer "B.Cu") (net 4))
 (segment (start 153.147158 56.599999) (end 151.547159 55) (width 0.2) (layer "B.Cu") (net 4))
 (segment (start 148.047157 55) (end 145.647158 57.399999) (width 0.2) (layer "B.Cu") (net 4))
 (segment (start 151.547159 55) (end 148.047157 55) (width 0.2) (layer "B.Cu") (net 4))
 (segment (start 135 57.5) (end 137.58 54.92) (width 0.2) (layer "B.Cu") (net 4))
 (segment (start 132.5 65.08) (end 135 62.58) (width 0.2) (layer "B.Cu") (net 4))
 (segment (start 91.38 56.19) (end 84.92375 56.19) (width 0.2) (layer "B.Cu") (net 4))
 (segment (start 102.5 60) (end 127.42 60) (width 0.2) (layer "B.Cu") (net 4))
 (segment (start 99 63.81) (end 91.38 56.19) (width 0.2) (layer "B.Cu") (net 4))
 (segment (start 81.12125 52.3875) (end 84.92375 56.19) (width 0.2) (layer "B.Cu") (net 4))
 (segment (start 94.28912 48.302) (end 91.28125 51.30987) (width 0.2) (layer "F.Cu") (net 11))
 (segment (start 126.18 52.38) (end 132.5 52.38) (width 0.2) (layer "F.Cu") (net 11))
 (segment (start 109.6678 48.302) (end 117.902 48.302) (width 0.2) (layer "F.Cu") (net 11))
 (segment (start 91.28125 51.30987) (end 91.28125 52.3875) (width 0.2) (layer "F.Cu") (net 11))
 (segment (start 109.6678 48.302) (end 94.28912 48.302) (width 0.2) (layer "F.Cu") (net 11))
 (segment (start 117.902 48.302) (end 120.8 51.2) (width 0.2) (layer "F.Cu") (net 11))
 (segment (start 125 51.2) (end 126.18 52.38) (width 0.2) (layer "F.Cu") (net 11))
 (via (at 120.8 51.2) (size 0.6) (drill 0.3) (layers "F.Cu" "B.Cu") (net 11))
 (via (at 125 51.2) (size 0.6) (drill 0.3) (layers "F.Cu" "B.Cu") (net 11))
 (segment (start 125 51.2) (end 120.8 51.2) (width 0.2) (layer "B.Cu") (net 11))
 (segment (start 120 47.5) (end 90.25375 47.5) (width 0.2) (layer "F.Cu") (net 13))
 (segment (start 132.5 60) (end 120 47.5) (width 0.2) (layer "F.Cu") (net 13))
 (segment (start 86.20125 51.5525) (end 86.20125 52.3875) (width 0.2) (layer "F.Cu") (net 13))
 (segment (start 90.25375 47.5) (end 86.20125 51.5525) (width 0.2) (layer "F.Cu") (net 13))
 (segment (start 129.24 54.2) (end 127.8 54.2) (width 0.2) (layer "F.Cu") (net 12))
 (segment (start 88.74125 49.5796) (end 88.74125 52.3875) (width 0.2) (layer "F.Cu") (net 12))
 (segment (start 132.5 57.46) (end 129.24 54.2) (width 0.2) (layer "F.Cu") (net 12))
 (segment (start 119.501 47.901) (end 90.41985 47.901) (width 0.2) (layer "F.Cu") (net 12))
 (segment (start 90.41985 47.901) (end 88.74125 49.5796) (width 0.2) (layer "F.Cu") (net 12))
 (segment (start 125.8 54.2) (end 119.501 47.901) (width 0.2) (layer "F.Cu") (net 12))
 (via (at 125.8 54.2) (size 0.6) (drill 0.3) (layers "F.Cu" "B.Cu") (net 12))
 (via (at 127.8 54.2) (size 0.6) (drill 0.3) (layers "F.Cu" "B.Cu") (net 12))
 (segment (start 127.8 54.2) (end 125.8 54.2) (width 0.2) (layer "B.Cu") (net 12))
 (segment (start 82.5 52.5) (end 82.6125 52.3875) (width 0.2) (layer "F.Cu") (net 3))
 (segment (start 93.2 58.2) (end 92.6 58.8) (width 0.2) (layer "F.Cu") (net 3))
 (segment (start 117.5 62.5) (end 117.5 57.5) (width 0.2) (layer "F.Cu") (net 3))
 (segment (start 82.6125 52.3875) (end 83.66125 52.3875) (width 0.2) (layer "F.Cu") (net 3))
 (segment (start 95 58.2) (end 93.2 58.2) (width 0.2) (layer "F.Cu") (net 3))
 (segment (start 82.5 55) (end 82.5 52.5) (width 0.2) (layer "F.Cu") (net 3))
 (via (at 82.5 55) (size 0.6) (drill 0.3) (layers "F.Cu" "B.Cu") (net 3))
 (via (at 117.5 57.5) (size 0.6) (drill 0.3) (layers "F.Cu" "B.Cu") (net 3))
 (via (at 95 58.2) (size 0.6) (drill 0.3) (layers "F.Cu" "B.Cu") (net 3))
 (via (at 92.6 58.8) (size 0.6) (drill 0.3) (layers "F.Cu" "B.Cu") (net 3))
 (via (at 117.5 62.5) (size 0.6) (drill 0.3) (layers "F.Cu" "B.Cu") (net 3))
 (segment (start 127.38 62.5) (end 117.5 62.5) (width 0.2) (layer "B.Cu") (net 3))
 (segment (start 99 61.27) (end 95.93 58.2) (width 0.2) (layer "B.Cu") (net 3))
 (segment (start 117.5 57.5) (end 102.77 57.5) (width 0.2) (layer "B.Cu") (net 3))
 (segment (start 132.5 67.62) (end 127.38 62.5) (width 0.2) (layer "B.Cu") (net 3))
 (segment (start 102.77 57.5) (end 99 61.27) (width 0.2) (layer "B.Cu") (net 3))
 (segment (start 92.53 58.73) (end 86.23 58.73) (width 0.2) (layer "B.Cu") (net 3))
 (segment (start 92.6 58.8) (end 92.53 58.73) (width 0.2) (layer "B.Cu") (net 3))
 (segment (start 86.23 58.73) (end 82.5 55) (width 0.2) (layer "B.Cu") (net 3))
 (segment (start 95.93 58.2) (end 95 58.2) (width 0.2) (layer "B.Cu") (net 3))
 (segment (start 93.82125 67.6275) (end 93.82125 61.36875) (width 0.2) (layer "F.Cu") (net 1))
 (segment (start 93.82125 61.36875) (end 99 56.19) (width 0.2) (layer "F.Cu") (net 1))
 (segment (start 102.27 58.73) (end 102.6 58.4) (width 0.2) (layer "F.Cu") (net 2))
 (segment (start 101.7875 52.3875) (end 93.82125 52.3875) (width 0.2) (layer "F.Cu") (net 2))
 (segment (start 99 58.73) (end 102.27 58.73) (width 0.2) (layer "F.Cu") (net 2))
 (segment (start 102.6 53.2) (end 101.7875 52.3875) (width 0.2) (layer "F.Cu") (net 2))
 (segment (start 102.6 58.4) (end 102.6 53.2) (width 0.2) (layer "F.Cu") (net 2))
 (segment (start 151.647158 57.399999) (end 150.100001 57.399999) (width 0.2) (layer "B.Cu") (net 16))
 (segment (start 146.900001 62.599999) (end 145.647158 62.599999) (width 0.2) (layer "B.Cu") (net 16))
 (segment (start 147.5 60) (end 147.5 62) (width 0.2) (layer "B.Cu") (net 16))
 (segment (start 147.5 62) (end 146.900001 62.599999) (width 0.2) (layer "B.Cu") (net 16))
 (segment (start 150.100001 57.399999) (end 147.5 60) (width 0.2) (layer "B.Cu") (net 16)))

